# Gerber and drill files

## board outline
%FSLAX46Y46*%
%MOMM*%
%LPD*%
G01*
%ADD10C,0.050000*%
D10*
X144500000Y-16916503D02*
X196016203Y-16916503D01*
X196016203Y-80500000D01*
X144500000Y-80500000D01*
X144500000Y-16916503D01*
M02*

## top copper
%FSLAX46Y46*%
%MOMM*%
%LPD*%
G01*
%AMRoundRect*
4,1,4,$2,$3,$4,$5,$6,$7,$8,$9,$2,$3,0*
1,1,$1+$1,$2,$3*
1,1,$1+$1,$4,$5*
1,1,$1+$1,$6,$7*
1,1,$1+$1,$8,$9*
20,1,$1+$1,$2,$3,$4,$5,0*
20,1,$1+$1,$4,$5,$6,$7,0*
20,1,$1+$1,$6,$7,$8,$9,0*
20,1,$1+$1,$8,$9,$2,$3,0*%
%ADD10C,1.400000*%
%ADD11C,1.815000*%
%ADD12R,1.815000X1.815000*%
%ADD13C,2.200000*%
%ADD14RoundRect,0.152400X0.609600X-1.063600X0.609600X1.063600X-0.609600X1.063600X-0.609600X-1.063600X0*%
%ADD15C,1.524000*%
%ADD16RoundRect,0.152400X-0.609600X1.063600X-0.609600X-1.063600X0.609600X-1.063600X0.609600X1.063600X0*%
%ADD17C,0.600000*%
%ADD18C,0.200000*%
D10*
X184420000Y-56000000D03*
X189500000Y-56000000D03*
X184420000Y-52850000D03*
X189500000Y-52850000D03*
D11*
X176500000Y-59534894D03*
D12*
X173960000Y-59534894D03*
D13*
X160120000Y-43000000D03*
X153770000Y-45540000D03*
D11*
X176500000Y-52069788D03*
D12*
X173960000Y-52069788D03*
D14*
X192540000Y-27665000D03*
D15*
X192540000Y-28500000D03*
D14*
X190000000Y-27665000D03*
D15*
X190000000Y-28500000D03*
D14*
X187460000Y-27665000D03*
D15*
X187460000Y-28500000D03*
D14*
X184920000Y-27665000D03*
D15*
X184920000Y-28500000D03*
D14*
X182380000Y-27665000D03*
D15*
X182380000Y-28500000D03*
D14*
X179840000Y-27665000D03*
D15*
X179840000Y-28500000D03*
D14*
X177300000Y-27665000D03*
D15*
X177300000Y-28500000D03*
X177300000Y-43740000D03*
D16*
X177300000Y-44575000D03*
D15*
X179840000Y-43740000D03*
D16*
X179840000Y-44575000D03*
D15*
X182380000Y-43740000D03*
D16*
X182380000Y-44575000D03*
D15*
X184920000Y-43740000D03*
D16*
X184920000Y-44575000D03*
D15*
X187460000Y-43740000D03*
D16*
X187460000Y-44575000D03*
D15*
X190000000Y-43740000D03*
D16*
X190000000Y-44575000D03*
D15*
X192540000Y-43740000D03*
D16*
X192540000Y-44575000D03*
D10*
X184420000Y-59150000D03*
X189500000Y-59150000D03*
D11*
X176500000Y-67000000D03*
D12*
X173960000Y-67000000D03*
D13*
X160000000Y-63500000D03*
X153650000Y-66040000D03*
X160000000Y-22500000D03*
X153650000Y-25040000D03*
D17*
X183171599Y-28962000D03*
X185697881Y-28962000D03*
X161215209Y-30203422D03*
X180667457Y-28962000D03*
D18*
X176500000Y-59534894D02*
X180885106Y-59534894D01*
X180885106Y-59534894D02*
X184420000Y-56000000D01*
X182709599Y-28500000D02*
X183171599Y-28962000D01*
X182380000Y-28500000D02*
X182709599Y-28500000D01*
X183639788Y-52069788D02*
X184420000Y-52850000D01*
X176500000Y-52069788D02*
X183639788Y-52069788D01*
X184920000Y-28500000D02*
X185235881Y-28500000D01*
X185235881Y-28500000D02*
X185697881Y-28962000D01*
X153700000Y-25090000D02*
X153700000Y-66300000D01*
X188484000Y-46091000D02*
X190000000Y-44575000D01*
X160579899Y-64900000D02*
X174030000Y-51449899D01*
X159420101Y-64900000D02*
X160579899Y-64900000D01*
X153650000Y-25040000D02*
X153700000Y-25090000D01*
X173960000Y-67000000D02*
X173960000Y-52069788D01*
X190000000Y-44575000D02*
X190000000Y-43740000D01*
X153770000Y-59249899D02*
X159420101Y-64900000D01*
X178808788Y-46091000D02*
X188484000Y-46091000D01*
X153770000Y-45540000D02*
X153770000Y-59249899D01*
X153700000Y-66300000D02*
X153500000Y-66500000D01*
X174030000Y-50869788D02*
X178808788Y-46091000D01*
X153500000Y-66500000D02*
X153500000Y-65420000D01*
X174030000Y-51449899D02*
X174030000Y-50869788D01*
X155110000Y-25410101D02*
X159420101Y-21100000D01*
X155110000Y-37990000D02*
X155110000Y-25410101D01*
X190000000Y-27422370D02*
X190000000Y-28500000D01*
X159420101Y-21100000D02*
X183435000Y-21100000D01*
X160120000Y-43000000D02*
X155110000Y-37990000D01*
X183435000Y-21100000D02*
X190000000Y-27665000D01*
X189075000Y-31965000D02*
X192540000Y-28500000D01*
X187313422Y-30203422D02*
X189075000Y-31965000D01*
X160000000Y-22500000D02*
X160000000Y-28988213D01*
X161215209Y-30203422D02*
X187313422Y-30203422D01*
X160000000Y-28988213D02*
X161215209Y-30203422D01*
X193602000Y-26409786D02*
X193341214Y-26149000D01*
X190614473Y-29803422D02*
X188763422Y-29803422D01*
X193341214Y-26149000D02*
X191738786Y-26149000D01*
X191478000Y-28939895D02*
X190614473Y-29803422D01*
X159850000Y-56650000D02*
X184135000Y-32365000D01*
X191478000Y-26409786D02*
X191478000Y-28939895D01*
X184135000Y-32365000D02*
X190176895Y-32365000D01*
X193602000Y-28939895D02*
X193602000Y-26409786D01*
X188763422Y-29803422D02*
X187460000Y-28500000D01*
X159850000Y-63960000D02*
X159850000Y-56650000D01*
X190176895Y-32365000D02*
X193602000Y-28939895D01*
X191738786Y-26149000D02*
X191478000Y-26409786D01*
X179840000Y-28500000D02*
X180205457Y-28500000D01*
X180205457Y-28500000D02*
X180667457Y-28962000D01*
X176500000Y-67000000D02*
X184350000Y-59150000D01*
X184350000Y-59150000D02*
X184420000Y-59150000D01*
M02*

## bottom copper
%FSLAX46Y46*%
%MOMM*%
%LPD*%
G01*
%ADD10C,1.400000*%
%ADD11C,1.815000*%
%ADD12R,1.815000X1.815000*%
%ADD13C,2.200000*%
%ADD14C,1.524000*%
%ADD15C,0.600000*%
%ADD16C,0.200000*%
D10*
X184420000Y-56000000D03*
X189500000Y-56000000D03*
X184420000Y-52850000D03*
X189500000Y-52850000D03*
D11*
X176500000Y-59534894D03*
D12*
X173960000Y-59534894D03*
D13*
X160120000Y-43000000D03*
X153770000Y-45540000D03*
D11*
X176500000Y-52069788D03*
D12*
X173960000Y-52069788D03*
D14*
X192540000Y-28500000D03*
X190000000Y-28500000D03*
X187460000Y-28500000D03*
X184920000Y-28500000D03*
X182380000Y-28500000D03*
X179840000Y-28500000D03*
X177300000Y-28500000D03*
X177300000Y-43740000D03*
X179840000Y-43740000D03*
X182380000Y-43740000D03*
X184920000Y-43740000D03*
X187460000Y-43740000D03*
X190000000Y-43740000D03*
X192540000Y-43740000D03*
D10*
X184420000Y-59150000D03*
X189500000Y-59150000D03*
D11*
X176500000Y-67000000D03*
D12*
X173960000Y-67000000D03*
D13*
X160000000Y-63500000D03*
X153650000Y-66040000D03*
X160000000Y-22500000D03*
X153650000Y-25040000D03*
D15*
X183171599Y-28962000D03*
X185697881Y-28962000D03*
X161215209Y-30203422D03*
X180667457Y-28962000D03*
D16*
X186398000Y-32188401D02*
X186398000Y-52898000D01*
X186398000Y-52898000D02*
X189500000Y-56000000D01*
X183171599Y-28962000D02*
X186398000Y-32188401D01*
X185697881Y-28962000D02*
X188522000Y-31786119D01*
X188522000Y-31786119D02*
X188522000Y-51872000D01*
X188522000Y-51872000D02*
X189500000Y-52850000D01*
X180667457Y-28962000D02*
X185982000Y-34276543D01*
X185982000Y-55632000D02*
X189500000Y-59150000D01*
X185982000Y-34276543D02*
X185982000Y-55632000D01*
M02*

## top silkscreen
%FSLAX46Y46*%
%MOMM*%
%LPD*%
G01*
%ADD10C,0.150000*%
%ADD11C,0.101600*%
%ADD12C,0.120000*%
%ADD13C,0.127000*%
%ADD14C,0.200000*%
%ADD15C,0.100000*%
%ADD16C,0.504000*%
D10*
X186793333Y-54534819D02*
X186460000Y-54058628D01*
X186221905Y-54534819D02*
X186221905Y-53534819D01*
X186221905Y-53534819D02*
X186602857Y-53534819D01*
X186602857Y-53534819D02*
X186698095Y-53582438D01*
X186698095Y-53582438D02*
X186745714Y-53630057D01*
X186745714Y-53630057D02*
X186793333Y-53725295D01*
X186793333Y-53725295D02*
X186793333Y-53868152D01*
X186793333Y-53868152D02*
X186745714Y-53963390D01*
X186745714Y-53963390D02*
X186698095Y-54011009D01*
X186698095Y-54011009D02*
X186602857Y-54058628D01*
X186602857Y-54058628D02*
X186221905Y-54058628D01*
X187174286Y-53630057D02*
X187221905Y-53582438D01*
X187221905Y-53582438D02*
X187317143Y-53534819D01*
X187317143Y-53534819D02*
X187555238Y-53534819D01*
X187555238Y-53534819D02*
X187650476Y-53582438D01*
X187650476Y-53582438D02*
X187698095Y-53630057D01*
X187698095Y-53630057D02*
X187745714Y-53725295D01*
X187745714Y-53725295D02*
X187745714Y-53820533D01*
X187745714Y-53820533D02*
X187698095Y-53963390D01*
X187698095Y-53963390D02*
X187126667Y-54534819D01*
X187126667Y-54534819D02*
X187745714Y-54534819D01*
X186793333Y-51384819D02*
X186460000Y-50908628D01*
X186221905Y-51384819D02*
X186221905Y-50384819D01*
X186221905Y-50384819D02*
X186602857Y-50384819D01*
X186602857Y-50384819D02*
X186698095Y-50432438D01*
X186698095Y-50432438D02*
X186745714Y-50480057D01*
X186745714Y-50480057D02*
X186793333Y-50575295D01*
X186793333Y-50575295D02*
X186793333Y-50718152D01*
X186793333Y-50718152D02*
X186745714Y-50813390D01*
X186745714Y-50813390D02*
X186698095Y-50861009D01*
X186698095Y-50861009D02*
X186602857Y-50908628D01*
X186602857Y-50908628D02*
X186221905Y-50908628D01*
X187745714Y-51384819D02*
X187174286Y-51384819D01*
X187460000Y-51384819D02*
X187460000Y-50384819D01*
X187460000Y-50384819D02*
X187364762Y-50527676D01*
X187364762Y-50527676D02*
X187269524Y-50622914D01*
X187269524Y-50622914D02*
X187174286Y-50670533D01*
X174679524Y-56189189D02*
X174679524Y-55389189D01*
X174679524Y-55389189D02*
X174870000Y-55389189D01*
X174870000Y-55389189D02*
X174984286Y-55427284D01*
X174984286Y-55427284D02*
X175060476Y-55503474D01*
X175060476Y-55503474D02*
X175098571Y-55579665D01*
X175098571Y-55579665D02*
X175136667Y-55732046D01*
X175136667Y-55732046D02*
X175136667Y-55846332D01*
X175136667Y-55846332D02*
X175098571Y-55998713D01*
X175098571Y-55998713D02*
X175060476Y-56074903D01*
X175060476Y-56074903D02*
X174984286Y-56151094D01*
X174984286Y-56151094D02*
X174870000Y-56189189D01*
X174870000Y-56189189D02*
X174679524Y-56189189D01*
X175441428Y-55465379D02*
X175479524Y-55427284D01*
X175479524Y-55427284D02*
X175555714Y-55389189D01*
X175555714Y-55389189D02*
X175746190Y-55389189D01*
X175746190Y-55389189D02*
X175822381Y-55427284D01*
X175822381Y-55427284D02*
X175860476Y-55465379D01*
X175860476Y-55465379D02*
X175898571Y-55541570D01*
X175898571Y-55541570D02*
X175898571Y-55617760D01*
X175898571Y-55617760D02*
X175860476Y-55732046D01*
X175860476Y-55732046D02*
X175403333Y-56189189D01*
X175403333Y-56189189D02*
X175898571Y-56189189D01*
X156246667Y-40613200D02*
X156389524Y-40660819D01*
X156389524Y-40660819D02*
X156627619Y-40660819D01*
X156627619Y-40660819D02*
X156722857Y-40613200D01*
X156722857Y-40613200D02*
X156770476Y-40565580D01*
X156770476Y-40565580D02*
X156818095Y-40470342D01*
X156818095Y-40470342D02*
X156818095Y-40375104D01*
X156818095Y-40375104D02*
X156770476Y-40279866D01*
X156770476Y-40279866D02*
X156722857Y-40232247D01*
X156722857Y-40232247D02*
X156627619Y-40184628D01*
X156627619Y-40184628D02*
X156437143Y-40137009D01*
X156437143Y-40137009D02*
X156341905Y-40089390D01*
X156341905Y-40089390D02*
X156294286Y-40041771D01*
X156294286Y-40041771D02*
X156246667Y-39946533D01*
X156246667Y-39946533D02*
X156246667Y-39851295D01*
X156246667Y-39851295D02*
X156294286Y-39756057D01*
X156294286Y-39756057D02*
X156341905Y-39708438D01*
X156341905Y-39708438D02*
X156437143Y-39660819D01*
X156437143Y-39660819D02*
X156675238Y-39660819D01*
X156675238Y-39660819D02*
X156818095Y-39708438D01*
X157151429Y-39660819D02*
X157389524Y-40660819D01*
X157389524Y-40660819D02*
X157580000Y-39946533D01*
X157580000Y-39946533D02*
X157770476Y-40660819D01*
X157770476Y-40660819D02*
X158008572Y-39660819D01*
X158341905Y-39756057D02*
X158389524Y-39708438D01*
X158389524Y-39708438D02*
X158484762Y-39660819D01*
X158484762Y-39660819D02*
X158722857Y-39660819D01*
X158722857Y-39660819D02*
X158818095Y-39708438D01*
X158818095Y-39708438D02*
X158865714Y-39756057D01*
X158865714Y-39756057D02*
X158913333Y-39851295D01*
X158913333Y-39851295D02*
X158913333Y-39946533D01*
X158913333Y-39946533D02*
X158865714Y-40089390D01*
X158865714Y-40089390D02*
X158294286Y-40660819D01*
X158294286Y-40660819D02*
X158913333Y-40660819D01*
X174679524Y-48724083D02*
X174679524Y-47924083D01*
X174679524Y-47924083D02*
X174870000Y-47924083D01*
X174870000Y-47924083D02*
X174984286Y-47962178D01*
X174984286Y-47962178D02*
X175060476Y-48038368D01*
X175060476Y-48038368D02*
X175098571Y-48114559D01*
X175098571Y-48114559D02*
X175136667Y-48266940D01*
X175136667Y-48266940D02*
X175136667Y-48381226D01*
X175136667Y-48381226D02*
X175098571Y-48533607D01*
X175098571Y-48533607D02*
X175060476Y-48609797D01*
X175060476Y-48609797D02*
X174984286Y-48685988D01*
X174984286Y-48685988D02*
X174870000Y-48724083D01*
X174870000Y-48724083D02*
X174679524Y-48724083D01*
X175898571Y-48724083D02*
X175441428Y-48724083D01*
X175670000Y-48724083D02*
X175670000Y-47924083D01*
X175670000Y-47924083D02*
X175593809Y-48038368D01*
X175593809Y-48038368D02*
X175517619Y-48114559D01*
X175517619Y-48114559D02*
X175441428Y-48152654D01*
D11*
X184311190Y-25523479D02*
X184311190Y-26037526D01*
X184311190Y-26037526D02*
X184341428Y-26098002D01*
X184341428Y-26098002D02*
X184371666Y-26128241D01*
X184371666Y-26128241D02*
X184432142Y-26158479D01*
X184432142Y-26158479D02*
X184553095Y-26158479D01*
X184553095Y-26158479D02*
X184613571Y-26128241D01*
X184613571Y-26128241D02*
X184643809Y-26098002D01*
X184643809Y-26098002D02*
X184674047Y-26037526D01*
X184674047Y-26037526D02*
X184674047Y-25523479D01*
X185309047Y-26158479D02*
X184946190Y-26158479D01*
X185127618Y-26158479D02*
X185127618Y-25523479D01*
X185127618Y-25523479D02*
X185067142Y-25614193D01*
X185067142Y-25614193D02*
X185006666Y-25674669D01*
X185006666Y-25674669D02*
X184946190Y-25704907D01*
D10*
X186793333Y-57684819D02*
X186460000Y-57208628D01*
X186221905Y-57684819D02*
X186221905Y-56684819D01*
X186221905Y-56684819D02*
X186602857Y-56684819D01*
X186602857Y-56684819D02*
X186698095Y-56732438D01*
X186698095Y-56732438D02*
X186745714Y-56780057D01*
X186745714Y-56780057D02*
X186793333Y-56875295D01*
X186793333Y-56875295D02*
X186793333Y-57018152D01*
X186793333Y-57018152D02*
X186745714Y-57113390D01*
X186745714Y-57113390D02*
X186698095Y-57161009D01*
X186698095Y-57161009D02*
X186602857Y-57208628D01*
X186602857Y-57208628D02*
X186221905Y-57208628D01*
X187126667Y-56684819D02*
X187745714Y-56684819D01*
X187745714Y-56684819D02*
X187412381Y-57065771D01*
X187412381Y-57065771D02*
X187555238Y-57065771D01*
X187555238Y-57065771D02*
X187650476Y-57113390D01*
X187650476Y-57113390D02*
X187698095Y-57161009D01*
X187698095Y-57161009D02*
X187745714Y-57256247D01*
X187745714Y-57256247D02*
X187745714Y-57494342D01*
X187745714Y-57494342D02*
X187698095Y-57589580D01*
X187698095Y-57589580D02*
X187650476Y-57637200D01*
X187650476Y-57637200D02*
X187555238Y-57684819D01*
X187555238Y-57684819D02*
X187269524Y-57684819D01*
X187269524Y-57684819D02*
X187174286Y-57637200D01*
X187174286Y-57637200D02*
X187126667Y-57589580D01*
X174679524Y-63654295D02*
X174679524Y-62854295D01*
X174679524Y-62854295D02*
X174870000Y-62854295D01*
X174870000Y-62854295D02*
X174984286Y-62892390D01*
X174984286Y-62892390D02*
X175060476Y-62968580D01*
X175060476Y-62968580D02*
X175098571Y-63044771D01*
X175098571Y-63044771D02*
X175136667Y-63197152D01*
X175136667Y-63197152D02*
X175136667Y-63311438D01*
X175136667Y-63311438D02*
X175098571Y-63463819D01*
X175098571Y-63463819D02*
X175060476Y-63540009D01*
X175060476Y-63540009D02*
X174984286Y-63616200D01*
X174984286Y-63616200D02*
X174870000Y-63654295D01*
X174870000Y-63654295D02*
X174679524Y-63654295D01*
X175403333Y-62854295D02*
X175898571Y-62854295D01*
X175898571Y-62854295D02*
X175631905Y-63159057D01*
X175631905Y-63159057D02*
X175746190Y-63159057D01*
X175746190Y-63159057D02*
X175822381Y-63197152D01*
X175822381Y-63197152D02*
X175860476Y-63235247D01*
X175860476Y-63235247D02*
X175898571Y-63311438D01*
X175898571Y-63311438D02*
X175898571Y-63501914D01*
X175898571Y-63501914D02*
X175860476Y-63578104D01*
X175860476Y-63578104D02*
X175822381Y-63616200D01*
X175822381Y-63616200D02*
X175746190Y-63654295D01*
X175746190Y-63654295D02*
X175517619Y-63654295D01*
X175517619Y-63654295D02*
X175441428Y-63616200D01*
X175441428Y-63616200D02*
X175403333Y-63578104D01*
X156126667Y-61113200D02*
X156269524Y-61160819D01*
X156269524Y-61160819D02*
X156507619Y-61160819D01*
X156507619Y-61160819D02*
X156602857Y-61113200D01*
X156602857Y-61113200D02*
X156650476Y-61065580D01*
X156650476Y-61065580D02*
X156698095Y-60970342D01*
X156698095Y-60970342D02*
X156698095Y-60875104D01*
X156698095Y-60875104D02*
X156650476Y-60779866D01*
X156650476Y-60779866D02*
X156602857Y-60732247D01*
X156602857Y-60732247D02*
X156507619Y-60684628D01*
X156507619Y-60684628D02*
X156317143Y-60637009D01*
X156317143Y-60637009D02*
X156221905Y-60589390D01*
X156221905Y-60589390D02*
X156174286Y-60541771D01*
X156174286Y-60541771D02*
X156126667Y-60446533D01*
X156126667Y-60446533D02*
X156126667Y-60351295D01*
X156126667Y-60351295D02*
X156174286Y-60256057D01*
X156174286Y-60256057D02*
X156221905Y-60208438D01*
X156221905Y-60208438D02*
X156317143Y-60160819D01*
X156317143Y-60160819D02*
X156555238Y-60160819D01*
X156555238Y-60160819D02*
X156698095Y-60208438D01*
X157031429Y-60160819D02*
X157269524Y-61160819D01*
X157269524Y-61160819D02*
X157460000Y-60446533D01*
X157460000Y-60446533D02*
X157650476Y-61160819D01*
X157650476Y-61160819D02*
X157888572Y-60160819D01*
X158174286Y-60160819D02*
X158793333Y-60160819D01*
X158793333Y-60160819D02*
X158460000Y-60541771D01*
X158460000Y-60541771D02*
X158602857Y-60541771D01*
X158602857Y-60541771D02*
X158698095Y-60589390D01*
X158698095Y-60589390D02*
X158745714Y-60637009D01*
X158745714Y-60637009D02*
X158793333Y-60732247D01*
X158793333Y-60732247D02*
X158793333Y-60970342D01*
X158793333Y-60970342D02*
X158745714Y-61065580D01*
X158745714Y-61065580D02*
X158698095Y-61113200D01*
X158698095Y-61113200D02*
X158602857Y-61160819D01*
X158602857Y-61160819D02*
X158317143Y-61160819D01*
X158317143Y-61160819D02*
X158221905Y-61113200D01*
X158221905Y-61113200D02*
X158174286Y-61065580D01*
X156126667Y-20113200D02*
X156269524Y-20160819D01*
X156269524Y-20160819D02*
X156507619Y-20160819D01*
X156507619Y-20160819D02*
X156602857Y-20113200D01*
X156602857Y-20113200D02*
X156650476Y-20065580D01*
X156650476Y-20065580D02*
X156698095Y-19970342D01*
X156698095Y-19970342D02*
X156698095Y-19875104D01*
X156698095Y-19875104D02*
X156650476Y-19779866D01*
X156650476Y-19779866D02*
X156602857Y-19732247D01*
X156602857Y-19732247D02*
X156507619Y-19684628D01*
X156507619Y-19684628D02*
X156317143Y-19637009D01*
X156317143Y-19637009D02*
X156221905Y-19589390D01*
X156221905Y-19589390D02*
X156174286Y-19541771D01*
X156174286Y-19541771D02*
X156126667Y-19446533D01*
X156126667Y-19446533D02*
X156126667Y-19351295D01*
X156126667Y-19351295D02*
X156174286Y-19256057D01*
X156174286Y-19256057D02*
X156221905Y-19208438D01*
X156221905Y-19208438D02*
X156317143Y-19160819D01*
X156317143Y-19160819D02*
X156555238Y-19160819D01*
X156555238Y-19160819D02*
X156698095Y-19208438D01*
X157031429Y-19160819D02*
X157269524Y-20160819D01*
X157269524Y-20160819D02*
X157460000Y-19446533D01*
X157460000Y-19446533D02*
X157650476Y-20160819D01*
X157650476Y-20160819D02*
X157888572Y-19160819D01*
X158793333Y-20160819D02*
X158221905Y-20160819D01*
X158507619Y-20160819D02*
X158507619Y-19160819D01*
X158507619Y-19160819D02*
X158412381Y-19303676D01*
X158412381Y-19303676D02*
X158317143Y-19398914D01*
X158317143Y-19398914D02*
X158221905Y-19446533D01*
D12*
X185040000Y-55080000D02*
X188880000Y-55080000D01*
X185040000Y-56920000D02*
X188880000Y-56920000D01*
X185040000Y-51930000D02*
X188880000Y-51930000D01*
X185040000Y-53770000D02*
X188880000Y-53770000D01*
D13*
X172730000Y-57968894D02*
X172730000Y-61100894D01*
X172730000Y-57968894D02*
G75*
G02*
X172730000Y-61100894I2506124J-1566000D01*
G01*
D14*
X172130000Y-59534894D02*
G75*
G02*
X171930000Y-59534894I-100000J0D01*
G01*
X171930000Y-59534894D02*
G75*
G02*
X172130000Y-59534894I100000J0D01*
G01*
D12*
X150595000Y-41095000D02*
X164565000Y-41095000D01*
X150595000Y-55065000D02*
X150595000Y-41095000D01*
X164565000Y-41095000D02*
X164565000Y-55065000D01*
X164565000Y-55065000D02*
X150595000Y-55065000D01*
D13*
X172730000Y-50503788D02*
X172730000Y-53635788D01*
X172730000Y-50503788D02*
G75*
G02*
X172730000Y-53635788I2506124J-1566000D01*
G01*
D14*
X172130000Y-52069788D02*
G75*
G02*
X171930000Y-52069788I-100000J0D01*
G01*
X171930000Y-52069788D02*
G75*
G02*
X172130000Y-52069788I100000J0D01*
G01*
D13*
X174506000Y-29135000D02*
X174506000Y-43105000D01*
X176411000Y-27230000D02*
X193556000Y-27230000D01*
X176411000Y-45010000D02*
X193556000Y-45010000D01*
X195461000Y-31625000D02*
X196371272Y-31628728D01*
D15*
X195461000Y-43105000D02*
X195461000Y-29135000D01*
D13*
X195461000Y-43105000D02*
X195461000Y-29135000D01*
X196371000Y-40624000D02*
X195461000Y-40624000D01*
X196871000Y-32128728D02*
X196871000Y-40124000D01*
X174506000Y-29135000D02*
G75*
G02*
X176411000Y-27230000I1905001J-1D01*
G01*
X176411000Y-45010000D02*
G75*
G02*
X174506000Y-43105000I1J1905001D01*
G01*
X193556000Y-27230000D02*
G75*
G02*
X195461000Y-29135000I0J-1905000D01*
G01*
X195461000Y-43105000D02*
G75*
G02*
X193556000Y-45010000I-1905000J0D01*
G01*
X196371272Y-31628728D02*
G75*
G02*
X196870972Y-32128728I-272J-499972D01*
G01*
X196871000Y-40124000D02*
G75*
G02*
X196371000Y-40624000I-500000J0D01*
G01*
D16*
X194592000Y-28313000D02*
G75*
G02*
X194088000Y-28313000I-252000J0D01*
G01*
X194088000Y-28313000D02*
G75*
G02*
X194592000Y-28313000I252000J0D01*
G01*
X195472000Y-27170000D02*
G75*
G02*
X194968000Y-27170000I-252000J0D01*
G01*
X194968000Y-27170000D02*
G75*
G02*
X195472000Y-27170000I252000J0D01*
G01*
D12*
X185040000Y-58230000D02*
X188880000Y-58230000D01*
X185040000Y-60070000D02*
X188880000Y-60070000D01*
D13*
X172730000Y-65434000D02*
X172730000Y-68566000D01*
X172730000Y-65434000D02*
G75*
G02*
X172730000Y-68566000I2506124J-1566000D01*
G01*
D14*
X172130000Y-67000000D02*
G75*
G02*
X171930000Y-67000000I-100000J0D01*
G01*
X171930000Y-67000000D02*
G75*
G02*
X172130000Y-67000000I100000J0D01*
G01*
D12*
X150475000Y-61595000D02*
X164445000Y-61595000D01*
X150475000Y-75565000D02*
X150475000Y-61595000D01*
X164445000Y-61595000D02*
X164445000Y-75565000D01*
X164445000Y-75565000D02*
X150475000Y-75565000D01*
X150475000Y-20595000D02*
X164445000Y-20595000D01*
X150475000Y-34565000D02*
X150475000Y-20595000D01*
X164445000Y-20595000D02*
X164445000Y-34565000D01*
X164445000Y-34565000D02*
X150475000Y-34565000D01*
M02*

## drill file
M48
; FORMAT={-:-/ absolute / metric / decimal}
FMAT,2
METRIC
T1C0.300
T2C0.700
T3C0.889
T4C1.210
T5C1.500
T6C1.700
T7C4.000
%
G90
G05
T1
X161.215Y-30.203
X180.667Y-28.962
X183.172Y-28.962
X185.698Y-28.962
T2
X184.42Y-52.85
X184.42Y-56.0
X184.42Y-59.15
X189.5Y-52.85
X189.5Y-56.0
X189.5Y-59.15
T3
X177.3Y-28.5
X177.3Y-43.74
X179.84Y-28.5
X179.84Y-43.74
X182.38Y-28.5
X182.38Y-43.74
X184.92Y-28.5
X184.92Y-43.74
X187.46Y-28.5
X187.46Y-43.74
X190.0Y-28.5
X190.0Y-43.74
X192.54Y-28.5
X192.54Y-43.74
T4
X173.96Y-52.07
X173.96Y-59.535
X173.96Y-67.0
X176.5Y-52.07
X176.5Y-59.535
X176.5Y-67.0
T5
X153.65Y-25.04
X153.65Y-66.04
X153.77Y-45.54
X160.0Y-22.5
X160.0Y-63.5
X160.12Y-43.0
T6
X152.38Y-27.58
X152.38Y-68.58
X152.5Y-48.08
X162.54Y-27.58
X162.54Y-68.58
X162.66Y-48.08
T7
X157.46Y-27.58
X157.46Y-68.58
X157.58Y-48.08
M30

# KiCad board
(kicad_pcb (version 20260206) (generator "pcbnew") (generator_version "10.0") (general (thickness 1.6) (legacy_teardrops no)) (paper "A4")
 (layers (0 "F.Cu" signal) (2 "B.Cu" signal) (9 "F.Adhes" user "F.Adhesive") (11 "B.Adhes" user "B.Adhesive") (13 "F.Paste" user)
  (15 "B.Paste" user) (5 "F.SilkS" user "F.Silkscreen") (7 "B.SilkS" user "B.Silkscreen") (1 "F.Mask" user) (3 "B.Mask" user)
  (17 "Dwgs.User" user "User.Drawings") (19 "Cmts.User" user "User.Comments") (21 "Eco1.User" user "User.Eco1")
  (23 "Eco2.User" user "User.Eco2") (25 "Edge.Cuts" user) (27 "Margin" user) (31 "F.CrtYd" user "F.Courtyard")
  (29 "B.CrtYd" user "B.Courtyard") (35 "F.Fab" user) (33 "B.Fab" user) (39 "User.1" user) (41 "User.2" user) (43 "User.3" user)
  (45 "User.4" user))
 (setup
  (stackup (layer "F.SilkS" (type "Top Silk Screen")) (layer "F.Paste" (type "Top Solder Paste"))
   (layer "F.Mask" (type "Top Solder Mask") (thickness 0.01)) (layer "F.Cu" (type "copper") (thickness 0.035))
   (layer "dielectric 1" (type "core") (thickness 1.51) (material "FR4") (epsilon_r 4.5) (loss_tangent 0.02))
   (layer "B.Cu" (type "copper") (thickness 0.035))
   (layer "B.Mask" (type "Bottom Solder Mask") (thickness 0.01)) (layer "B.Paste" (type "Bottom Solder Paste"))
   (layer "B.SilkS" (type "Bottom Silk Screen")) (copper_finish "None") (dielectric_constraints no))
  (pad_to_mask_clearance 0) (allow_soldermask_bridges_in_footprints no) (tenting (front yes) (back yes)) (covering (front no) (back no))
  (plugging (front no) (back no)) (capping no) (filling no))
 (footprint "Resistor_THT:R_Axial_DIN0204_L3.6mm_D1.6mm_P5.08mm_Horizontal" (layer "F.Cu") (at 184.42 56)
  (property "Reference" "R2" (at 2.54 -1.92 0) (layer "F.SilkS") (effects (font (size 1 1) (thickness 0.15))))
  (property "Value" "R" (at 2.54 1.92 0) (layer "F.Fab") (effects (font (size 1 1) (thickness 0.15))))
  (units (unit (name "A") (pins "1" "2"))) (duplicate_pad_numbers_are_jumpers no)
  (fp_line (start 0.62 -0.92) (end 4.46 -0.92) (stroke (width 0.12) (type solid)) (layer "F.SilkS"))
  (fp_line (start 0.62 0.92) (end 4.46 0.92) (stroke (width 0.12) (type solid)) (layer "F.SilkS"))
  (pad "1" thru_hole circle (at 0 0) (size 1.4 1.4) (drill 0.7) (layers "*.Cu" "*.Mask") (remove_unused_layers no) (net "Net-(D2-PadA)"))
  (pad "2" thru_hole circle (at 5.08 0) (size 1.4 1.4) (drill 0.7) (layers "*.Cu" "*.Mask") (remove_unused_layers no) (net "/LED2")))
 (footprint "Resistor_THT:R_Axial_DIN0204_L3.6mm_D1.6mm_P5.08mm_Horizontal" (layer "F.Cu") (at 184.42 52.85)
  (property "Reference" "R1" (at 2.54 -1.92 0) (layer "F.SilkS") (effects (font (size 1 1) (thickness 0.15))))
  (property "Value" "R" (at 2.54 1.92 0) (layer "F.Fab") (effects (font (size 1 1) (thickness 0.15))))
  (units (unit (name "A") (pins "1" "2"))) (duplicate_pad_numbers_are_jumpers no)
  (fp_line (start 0.62 -0.92) (end 4.46 -0.92) (stroke (width 0.12) (type solid)) (layer "F.SilkS"))
  (fp_line (start 0.62 0.92) (end 4.46 0.92) (stroke (width 0.12) (type solid)) (layer "F.SilkS"))
  (pad "1" thru_hole circle (at 0 0) (size 1.4 1.4) (drill 0.7) (layers "*.Cu" "*.Mask") (remove_unused_layers no) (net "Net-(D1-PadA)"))
  (pad "2" thru_hole circle (at 5.08 0) (size 1.4 1.4) (drill 0.7) (layers "*.Cu" "*.Mask") (remove_unused_layers no) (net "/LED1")))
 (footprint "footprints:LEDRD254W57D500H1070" (layer "F.Cu") (at 175.23 59.534894)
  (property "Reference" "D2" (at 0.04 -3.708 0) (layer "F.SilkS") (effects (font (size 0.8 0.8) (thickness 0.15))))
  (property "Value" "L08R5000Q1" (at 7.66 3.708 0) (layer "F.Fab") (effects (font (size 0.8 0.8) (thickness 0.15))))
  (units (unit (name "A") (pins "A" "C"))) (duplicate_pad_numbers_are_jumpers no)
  (fp_line (start -2.5 -1.566) (end -2.5 1.566) (stroke (width 0.127) (type solid)) (layer "F.SilkS"))
  (fp_arc (start -2.5 -1.566) (mid 2.961291 0) (end -2.5 1.566) (stroke (width 0.127) (type solid)) (layer "F.SilkS"))
  (fp_circle (center -3.2 0) (end -3.1 0) (stroke (width 0.2) (type solid)) (fill no) (layer "F.SilkS"))
  (pad "A" thru_hole circle (at 1.27 0) (size 1.815 1.815) (drill 1.21) (layers "*.Cu" "*.Mask") (remove_unused_layers no)
   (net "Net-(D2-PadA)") (solder_mask_margin 0.102))
  (pad "C" thru_hole rect (at -1.27 0) (size 1.815 1.815) (drill 1.21) (layers "*.Cu" "*.Mask") (remove_unused_layers no) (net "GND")
   (solder_mask_margin 0.102)))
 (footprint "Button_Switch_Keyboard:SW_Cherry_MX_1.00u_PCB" (layer "F.Cu") (at 160.12 43)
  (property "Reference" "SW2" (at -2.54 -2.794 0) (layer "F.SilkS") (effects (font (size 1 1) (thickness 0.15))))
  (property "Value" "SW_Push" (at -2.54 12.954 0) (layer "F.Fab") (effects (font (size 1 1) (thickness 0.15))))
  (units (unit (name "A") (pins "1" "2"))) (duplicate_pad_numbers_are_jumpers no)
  (fp_line (start -9.525 -1.905) (end 4.445 -1.905) (stroke (width 0.12) (type solid)) (layer "F.SilkS"))
  (fp_line (start -9.525 12.065) (end -9.525 -1.905) (stroke (width 0.12) (type solid)) (layer "F.SilkS"))
  (fp_line (start 4.445 -1.905) (end 4.445 12.065) (stroke (width 0.12) (type solid)) (layer "F.SilkS"))
  (fp_line (start 4.445 12.065) (end -9.525 12.065) (stroke (width 0.12) (type solid)) (layer "F.SilkS"))
  (pad "" np_thru_hole circle (at -7.62 5.08) (size 1.7 1.7) (drill 1.7) (layers "*.Cu" "*.Mask"))
  (pad "" np_thru_hole circle (at -2.54 5.08) (size 4 4) (drill 4) (layers "*.Cu" "*.Mask"))
  (pad "" np_thru_hole circle (at 2.54 5.08) (size 1.7 1.7) (drill 1.7) (layers "*.Cu" "*.Mask"))
  (pad "1" thru_hole circle (at 0 0) (size 2.2 2.2) (drill 1.5) (layers "*.Cu" "*.Mask") (remove_unused_layers no) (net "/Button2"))
  (pad "2" thru_hole circle (at -6.35 2.54) (size 2.2 2.2) (drill 1.5) (layers "*.Cu" "*.Mask") (remove_unused_layers no) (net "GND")))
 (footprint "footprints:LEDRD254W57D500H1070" (layer "F.Cu") (at 175.23 52.069788)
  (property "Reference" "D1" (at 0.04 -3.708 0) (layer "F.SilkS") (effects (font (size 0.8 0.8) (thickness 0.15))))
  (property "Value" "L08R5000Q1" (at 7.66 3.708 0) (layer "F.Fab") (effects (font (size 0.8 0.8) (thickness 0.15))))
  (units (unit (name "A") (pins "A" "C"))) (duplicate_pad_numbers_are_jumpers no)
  (fp_line (start -2.5 -1.566) (end -2.5 1.566) (stroke (width 0.127) (type solid)) (layer "F.SilkS"))
  (fp_arc (start -2.5 -1.566) (mid 2.961291 0) (end -2.5 1.566) (stroke (width 0.127) (type solid)) (layer "F.SilkS"))
  (fp_circle (center -3.2 0) (end -3.1 0) (stroke (width 0.2) (type solid)) (fill no) (layer "F.SilkS"))
  (pad "A" thru_hole circle (at 1.27 0) (size 1.815 1.815) (drill 1.21) (layers "*.Cu" "*.Mask") (remove_unused_layers no)
   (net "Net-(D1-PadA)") (solder_mask_margin 0.102))
  (pad "C" thru_hole rect (at -1.27 0) (size 1.815 1.815) (drill 1.21) (layers "*.Cu" "*.Mask") (remove_unused_layers no) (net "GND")
   (solder_mask_margin 0.102)))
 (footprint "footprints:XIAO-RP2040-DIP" (layer "F.Cu") (at 184.92 36.12)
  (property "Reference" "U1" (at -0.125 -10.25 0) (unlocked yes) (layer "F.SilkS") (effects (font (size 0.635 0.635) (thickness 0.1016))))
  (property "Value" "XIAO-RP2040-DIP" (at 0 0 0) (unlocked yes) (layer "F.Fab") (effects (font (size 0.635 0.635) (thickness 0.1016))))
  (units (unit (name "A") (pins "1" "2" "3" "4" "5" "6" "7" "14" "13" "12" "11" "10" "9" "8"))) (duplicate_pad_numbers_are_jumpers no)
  (fp_line (start -10.414 -6.985) (end -10.414 6.985) (stroke (width 0.127) (type solid)) (layer "F.SilkS"))
  (fp_line (start -8.509 -8.89) (end 8.636 -8.89) (stroke (width 0.127) (type solid)) (layer "F.SilkS"))
  (fp_line (start -8.509 8.89) (end 8.636 8.89) (stroke (width 0.127) (type solid)) (layer "F.SilkS"))
  (fp_line (start 10.541 -4.495) (end 11.451272 -4.491272) (stroke (width 0.127) (type solid)) (layer "F.SilkS"))
  (fp_line (start 10.541 6.985) (end 10.541 -6.985) (stroke (width 0.1) (type solid)) (layer "F.SilkS"))
  (fp_line (start 10.541 6.985) (end 10.541 -6.985) (stroke (width 0.127) (type solid)) (layer "F.SilkS"))
  (fp_line (start 11.451 4.504) (end 10.541 4.504) (stroke (width 0.127) (type solid)) (layer "F.SilkS"))
  (fp_line (start 11.951 -3.991272) (end 11.951 4.004) (stroke (width 0.127) (type solid)) (layer "F.SilkS"))
  (fp_arc (start -10.414 -6.985) (mid -9.856038 -8.332038) (end -8.509 -8.89) (stroke (width 0.127) (type solid)) (layer "F.SilkS"))
  (fp_arc (start -8.509 8.89) (mid -9.856038 8.332038) (end -10.414 6.985) (stroke (width 0.127) (type solid)) (layer "F.SilkS"))
  (fp_arc (start 8.636 -8.89) (mid 9.983038 -8.332038) (end 10.541 -6.985) (stroke (width 0.127) (type solid)) (layer "F.SilkS"))
  (fp_arc (start 10.541 6.985) (mid 9.983038 8.332038) (end 8.636 8.89) (stroke (width 0.127) (type solid)) (layer "F.SilkS"))
  (fp_arc (start 11.451272 -4.491272) (mid 11.804644 -4.344724) (end 11.951 -3.991272) (stroke (width 0.127) (type default))
   (layer "F.SilkS"))
  (fp_arc (start 11.951 4.004) (mid 11.804553 4.357553) (end 11.451 4.504) (stroke (width 0.127) (type default)) (layer "F.SilkS"))
  (fp_circle (center 9.42 -7.807) (end 9.674 -7.807) (stroke (width 0.5) (type solid)) (fill yes) (layer "F.SilkS"))
  (fp_circle (center 10.3 -8.95) (end 10.554 -8.95) (stroke (width 0.5) (type solid)) (fill yes) (layer "F.SilkS"))
  (pad "1" smd roundrect (at 7.62 -8.455 90) (size 2.432 1.524) (layers "F.Cu" "F.Mask") (roundrect_rratio 0.1) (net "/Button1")
   (thermal_bridge_angle 45))
  (pad "1" thru_hole circle (at 7.62 -7.62 90) (size 1.524 1.524) (drill 0.889) (layers "*.Cu" "*.Mask") (remove_unused_layers no)
   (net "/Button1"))
  (pad "2" smd roundrect (at 5.08 -8.455 90) (size 2.432 1.524) (layers "F.Cu" "F.Mask") (roundrect_rratio 0.1) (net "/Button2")
   (thermal_bridge_angle 45))
  (pad "2" thru_hole circle (at 5.08 -7.62 90) (size 1.524 1.524) (drill 0.889) (layers "*.Cu" "*.Mask") (remove_unused_layers no)
   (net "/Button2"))
  (pad "3" smd roundrect (at 2.54 -8.455 90) (size 2.432 1.524) (layers "F.Cu" "F.Mask") (roundrect_rratio 0.1) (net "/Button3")
   (thermal_bridge_angle 45))
  (pad "3" thru_hole circle (at 2.54 -7.62 90) (size 1.524 1.524) (drill 0.889) (layers "*.Cu" "*.Mask") (remove_unused_layers no)
   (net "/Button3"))
  (pad "4" smd roundrect (at 0 -8.455 90) (size 2.432 1.524) (layers "F.Cu" "F.Mask") (roundrect_rratio 0.1) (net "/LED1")
   (thermal_bridge_angle 45))
  (pad "4" thru_hole circle (at 0 -7.62 90) (size 1.524 1.524) (drill 0.889) (layers "*.Cu" "*.Mask") (remove_unused_layers no)
   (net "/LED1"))
  (pad "5" smd roundrect (at -2.54 -8.455 90) (size 2.432 1.524) (layers "F.Cu" "F.Mask") (roundrect_rratio 0.1) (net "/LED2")
   (thermal_bridge_angle 45))
  (pad "5" thru_hole circle (at -2.54 -7.62 90) (size 1.524 1.524) (drill 0.889) (layers "*.Cu" "*.Mask") (remove_unused_layers no)
   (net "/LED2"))
  (pad "6" smd roundrect (at -5.08 -8.455 90) (size 2.432 1.524) (layers "F.Cu" "F.Mask") (roundrect_rratio 0.1) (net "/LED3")
   (thermal_bridge_angle 45))
  (pad "6" thru_hole circle (at -5.08 -7.62 90) (size 1.524 1.524) (drill 0.889) (layers "*.Cu" "*.Mask") (remove_unused_layers no)
   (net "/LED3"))
  (pad "7" smd roundrect (at -7.62 -8.455 90) (size 2.432 1.524) (layers "F.Cu" "F.Mask") (roundrect_rratio 0.1)
   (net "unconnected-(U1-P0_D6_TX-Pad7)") (thermal_bridge_angle 45))
  (pad "7" thru_hole circle (at -7.62 -7.62 90) (size 1.524 1.524) (drill 0.889) (layers "*.Cu" "*.Mask") (remove_unused_layers no)
   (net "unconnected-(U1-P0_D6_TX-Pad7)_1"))
  (pad "8" thru_hole circle (at -7.62 7.62 270) (size 1.524 1.524) (drill 0.889) (layers "*.Cu" "*.Mask") (remove_unused_layers no)
   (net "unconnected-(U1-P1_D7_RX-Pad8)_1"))
  (pad "8" smd roundrect (at -7.62 8.455 270) (size 2.432 1.524) (layers "F.Cu" "F.Mask") (roundrect_rratio 0.1)
   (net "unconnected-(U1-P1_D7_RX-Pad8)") (thermal_bridge_angle 45))
  (pad "9" thru_hole circle (at -5.08 7.62 270) (size 1.524 1.524) (drill 0.889) (layers "*.Cu" "*.Mask") (remove_unused_layers no)
   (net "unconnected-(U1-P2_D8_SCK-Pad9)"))
  (pad "9" smd roundrect (at -5.08 8.455 270) (size 2.432 1.524) (layers "F.Cu" "F.Mask") (roundrect_rratio 0.1)
   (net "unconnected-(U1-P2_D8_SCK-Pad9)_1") (thermal_bridge_angle 45))
  (pad "10" thru_hole circle (at -2.54 7.62 270) (size 1.524 1.524) (drill 0.889) (layers "*.Cu" "*.Mask") (remove_unused_layers no)
   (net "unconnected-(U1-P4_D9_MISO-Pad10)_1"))
  (pad "10" smd roundrect (at -2.54 8.455 270) (size 2.432 1.524) (layers "F.Cu" "F.Mask") (roundrect_rratio 0.1)
   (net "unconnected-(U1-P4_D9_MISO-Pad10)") (thermal_bridge_angle 45))
  (pad "11" thru_hole circle (at 0 7.62 270) (size 1.524 1.524) (drill 0.889) (layers "*.Cu" "*.Mask") (remove_unused_layers no)
   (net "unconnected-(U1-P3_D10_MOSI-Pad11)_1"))
  (pad "11" smd roundrect (at 0 8.455 270) (size 2.432 1.524) (layers "F.Cu" "F.Mask") (roundrect_rratio 0.1)
   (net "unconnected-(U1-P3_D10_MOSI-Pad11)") (thermal_bridge_angle 45))
  (pad "12" thru_hole circle (at 2.54 7.62 270) (size 1.524 1.524) (drill 0.889) (layers "*.Cu" "*.Mask") (remove_unused_layers no)
   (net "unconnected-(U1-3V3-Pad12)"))
  (pad "12" smd roundrect (at 2.54 8.455 270) (size 2.432 1.524) (layers "F.Cu" "F.Mask") (roundrect_rratio 0.1)
   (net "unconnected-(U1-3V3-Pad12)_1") (thermal_bridge_angle 45))
  (pad "13" thru_hole circle (at 5.08 7.62 270) (size 1.524 1.524) (drill 0.889) (layers "*.Cu" "*.Mask") (remove_unused_layers no)
   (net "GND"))
  (pad "13" smd roundrect (at 5.08 8.455 270) (size 2.432 1.524) (layers "F.Cu" "F.Mask") (roundrect_rratio 0.1) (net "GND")
   (thermal_bridge_angle 45))
  (pad "14" thru_hole circle (at 7.62 7.62 270) (size 1.524 1.524) (drill 0.889) (layers "*.Cu" "*.Mask") (remove_unused_layers no)
   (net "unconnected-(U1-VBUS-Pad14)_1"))
  (pad "14" smd roundrect (at 7.62 8.455 270) (size 2.432 1.524) (layers "F.Cu" "F.Mask") (roundrect_rratio 0.1)
   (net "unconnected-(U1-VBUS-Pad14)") (thermal_bridge_angle 45)))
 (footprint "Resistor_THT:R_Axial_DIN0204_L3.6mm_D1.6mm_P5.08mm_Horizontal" (layer "F.Cu") (at 184.42 59.15)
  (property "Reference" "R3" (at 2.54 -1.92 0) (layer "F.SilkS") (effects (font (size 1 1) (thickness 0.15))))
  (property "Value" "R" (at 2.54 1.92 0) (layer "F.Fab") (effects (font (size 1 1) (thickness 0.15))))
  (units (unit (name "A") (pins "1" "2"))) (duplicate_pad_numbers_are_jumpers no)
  (fp_line (start 0.62 -0.92) (end 4.46 -0.92) (stroke (width 0.12) (type solid)) (layer "F.SilkS"))
  (fp_line (start 0.62 0.92) (end 4.46 0.92) (stroke (width 0.12) (type solid)) (layer "F.SilkS"))
  (pad "1" thru_hole circle (at 0 0) (size 1.4 1.4) (drill 0.7) (layers "*.Cu" "*.Mask") (remove_unused_layers no) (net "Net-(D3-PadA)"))
  (pad "2" thru_hole circle (at 5.08 0) (size 1.4 1.4) (drill 0.7) (layers "*.Cu" "*.Mask") (remove_unused_layers no) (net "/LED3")))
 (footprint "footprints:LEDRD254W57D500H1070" (layer "F.Cu") (at 175.23 67)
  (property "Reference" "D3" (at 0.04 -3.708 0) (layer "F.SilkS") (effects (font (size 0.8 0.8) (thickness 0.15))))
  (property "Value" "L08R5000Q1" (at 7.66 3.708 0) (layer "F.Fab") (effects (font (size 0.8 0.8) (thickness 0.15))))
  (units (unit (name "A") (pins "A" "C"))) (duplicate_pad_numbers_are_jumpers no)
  (fp_line (start -2.5 -1.566) (end -2.5 1.566) (stroke (width 0.127) (type solid)) (layer "F.SilkS"))
  (fp_arc (start -2.5 -1.566) (mid 2.961291 0) (end -2.5 1.566) (stroke (width 0.127) (type solid)) (layer "F.SilkS"))
  (fp_circle (center -3.2 0) (end -3.1 0) (stroke (width 0.2) (type solid)) (fill no) (layer "F.SilkS"))
  (pad "A" thru_hole circle (at 1.27 0) (size 1.815 1.815) (drill 1.21) (layers "*.Cu" "*.Mask") (remove_unused_layers no)
   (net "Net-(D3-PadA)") (solder_mask_margin 0.102))
  (pad "C" thru_hole rect (at -1.27 0) (size 1.815 1.815) (drill 1.21) (layers "*.Cu" "*.Mask") (remove_unused_layers no) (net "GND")
   (solder_mask_margin 0.102)))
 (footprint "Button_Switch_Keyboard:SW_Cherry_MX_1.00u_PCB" (layer "F.Cu") (at 160 63.5)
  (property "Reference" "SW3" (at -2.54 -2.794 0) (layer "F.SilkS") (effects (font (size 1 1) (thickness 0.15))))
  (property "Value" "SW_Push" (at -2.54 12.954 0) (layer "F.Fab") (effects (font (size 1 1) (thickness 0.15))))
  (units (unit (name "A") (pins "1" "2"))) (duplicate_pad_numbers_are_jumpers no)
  (fp_line (start -9.525 -1.905) (end 4.445 -1.905) (stroke (width 0.12) (type solid)) (layer "F.SilkS"))
  (fp_line (start -9.525 12.065) (end -9.525 -1.905) (stroke (width 0.12) (type solid)) (layer "F.SilkS"))
  (fp_line (start 4.445 -1.905) (end 4.445 12.065) (stroke (width 0.12) (type solid)) (layer "F.SilkS"))
  (fp_line (start 4.445 12.065) (end -9.525 12.065) (stroke (width 0.12) (type solid)) (layer "F.SilkS"))
  (pad "" np_thru_hole circle (at -7.62 5.08) (size 1.7 1.7) (drill 1.7) (layers "*.Cu" "*.Mask"))
  (pad "" np_thru_hole circle (at -2.54 5.08) (size 4 4) (drill 4) (layers "*.Cu" "*.Mask"))
  (pad "" np_thru_hole circle (at 2.54 5.08) (size 1.7 1.7) (drill 1.7) (layers "*.Cu" "*.Mask"))
  (pad "1" thru_hole circle (at 0 0) (size 2.2 2.2) (drill 1.5) (layers "*.Cu" "*.Mask") (remove_unused_layers no) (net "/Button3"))
  (pad "2" thru_hole circle (at -6.35 2.54) (size 2.2 2.2) (drill 1.5) (layers "*.Cu" "*.Mask") (remove_unused_layers no) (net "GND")))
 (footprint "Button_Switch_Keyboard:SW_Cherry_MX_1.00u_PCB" (layer "F.Cu") (at 160 22.5)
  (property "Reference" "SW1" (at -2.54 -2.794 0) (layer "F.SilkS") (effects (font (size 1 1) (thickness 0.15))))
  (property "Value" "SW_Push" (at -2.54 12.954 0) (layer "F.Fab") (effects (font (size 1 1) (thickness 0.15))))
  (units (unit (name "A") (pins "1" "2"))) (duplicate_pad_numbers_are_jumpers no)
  (fp_line (start -9.525 -1.905) (end 4.445 -1.905) (stroke (width 0.12) (type solid)) (layer "F.SilkS"))
  (fp_line (start -9.525 12.065) (end -9.525 -1.905) (stroke (width 0.12) (type solid)) (layer "F.SilkS"))
  (fp_line (start 4.445 -1.905) (end 4.445 12.065) (stroke (width 0.12) (type solid)) (layer "F.SilkS"))
  (fp_line (start 4.445 12.065) (end -9.525 12.065) (stroke (width 0.12) (type solid)) (layer "F.SilkS"))
  (pad "" np_thru_hole circle (at -7.62 5.08) (size 1.7 1.7) (drill 1.7) (layers "*.Cu" "*.Mask"))
  (pad "" np_thru_hole circle (at -2.54 5.08) (size 4 4) (drill 4) (layers "*.Cu" "*.Mask"))
  (pad "" np_thru_hole circle (at 2.54 5.08) (size 1.7 1.7) (drill 1.7) (layers "*.Cu" "*.Mask"))
  (pad "1" thru_hole circle (at 0 0) (size 2.2 2.2) (drill 1.5) (layers "*.Cu" "*.Mask") (remove_unused_layers no) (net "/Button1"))
  (pad "2" thru_hole circle (at -6.35 2.54) (size 2.2 2.2) (drill 1.5) (layers "*.Cu" "*.Mask") (remove_unused_layers no) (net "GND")))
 (gr_rect (start 144.5 16.916503) (end 196.016203 80.5) (stroke (width 0.05) (type default)) (fill no) (layer "Edge.Cuts"))
 (segment (start 176.5 59.534894) (end 180.885106 59.534894) (width 0.2) (layer "F.Cu") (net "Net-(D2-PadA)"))
 (segment (start 180.885106 59.534894) (end 184.42 56) (width 0.2) (layer "F.Cu") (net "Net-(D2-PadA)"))
 (segment (start 182.709599 28.5) (end 183.171599 28.962) (width 0.2) (layer "F.Cu") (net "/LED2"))
 (segment (start 182.38 28.5) (end 182.709599 28.5) (width 0.2) (layer "F.Cu") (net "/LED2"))
 (via (at 183.171599 28.962) (size 0.6) (drill 0.3) (layers "F.Cu" "B.Cu") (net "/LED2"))
 (segment (start 186.398 32.188401) (end 186.398 52.898) (width 0.2) (layer "B.Cu") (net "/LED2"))
 (segment (start 186.398 52.898) (end 189.5 56) (width 0.2) (layer "B.Cu") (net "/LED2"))
 (segment (start 183.171599 28.962) (end 186.398 32.188401) (width 0.2) (layer "B.Cu") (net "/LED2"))
 (segment (start 183.639788 52.069788) (end 184.42 52.85) (width 0.2) (layer "F.Cu") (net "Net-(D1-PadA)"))
 (segment (start 176.5 52.069788) (end 183.639788 52.069788) (width 0.2) (layer "F.Cu") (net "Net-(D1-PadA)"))
 (segment (start 184.92 28.5) (end 185.235881 28.5) (width 0.2) (layer "F.Cu") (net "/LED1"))
 (segment (start 185.235881 28.5) (end 185.697881 28.962) (width 0.2) (layer "F.Cu") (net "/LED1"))
 (via (at 185.697881 28.962) (size 0.6) (drill 0.3) (layers "F.Cu" "B.Cu") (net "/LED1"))
 (segment (start 185.697881 28.962) (end 188.522 31.786119) (width 0.2) (layer "B.Cu") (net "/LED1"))
 (segment (start 188.522 31.786119) (end 188.522 51.872) (width 0.2) (layer "B.Cu") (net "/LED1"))
 (segment (start 188.522 51.872) (end 189.5 52.85) (width 0.2) (layer "B.Cu") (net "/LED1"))
 (segment (start 153.7 25.09) (end 153.7 66.3) (width 0.2) (layer "F.Cu") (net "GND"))
 (segment (start 188.484 46.091) (end 190 44.575) (width 0.2) (layer "F.Cu") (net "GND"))
 (segment (start 160.579899 64.9) (end 174.03 51.449899) (width 0.2) (layer "F.Cu") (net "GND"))
 (segment (start 159.420101 64.9) (end 160.579899 64.9) (width 0.2) (layer "F.Cu") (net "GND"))
 (segment (start 153.65 25.04) (end 153.7 25.09) (width 0.2) (layer "F.Cu") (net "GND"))
 (segment (start 173.96 67) (end 173.96 52.069788) (width 0.2) (layer "F.Cu") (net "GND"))
 (segment (start 190 44.575) (end 190 43.74) (width 0.2) (layer "F.Cu") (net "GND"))
 (segment (start 153.77 59.249899) (end 159.420101 64.9) (width 0.2) (layer "F.Cu") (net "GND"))
 (segment (start 178.808788 46.091) (end 188.484 46.091) (width 0.2) (layer "F.Cu") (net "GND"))
 (segment (start 153.77 45.54) (end 153.77 59.249899) (width 0.2) (layer "F.Cu") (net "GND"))
 (segment (start 153.7 66.3) (end 153.5 66.5) (width 0.2) (layer "F.Cu") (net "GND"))
 (segment (start 174.03 50.869788) (end 178.808788 46.091) (width 0.2) (layer "F.Cu") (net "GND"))
 (segment (start 153.5 66.5) (end 153.5 65.42) (width 0.2) (layer "F.Cu") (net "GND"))
 (segment (start 174.03 51.449899) (end 174.03 50.869788) (width 0.2) (layer "F.Cu") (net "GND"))
 (segment (start 155.11 25.410101) (end 159.420101 21.1) (width 0.2) (layer "F.Cu") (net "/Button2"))
 (segment (start 155.11 37.99) (end 155.11 25.410101) (width 0.2) (layer "F.Cu") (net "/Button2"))
 (segment (start 190 27.42237) (end 190 28.5) (width 0.2) (layer "F.Cu") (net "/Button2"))
 (segment (start 159.420101 21.1) (end 183.435 21.1) (width 0.2) (layer "F.Cu") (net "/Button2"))
 (segment (start 160.12 43) (end 155.11 37.99) (width 0.2) (layer "F.Cu") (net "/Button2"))
 (segment (start 183.435 21.1) (end 190 27.665) (width 0.2) (layer "F.Cu") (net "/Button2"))
 (segment (start 189.075 31.965) (end 192.54 28.5) (width 0.2) (layer "F.Cu") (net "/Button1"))
 (segment (start 187.313422 30.203422) (end 189.075 31.965) (width 0.2) (layer "F.Cu") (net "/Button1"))
 (segment (start 160 22.5) (end 160 28.988213) (width 0.2) (layer "F.Cu") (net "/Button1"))
 (segment (start 161.215209 30.203422) (end 187.313422 30.203422) (width 0.2) (layer "F.Cu") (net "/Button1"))
 (segment (start 160 28.988213) (end 161.215209 30.203422) (width 0.2) (layer "F.Cu") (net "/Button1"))
 (via (at 161.215209 30.203422) (size 0.6) (drill 0.3) (layers "F.Cu" "B.Cu") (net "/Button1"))
 (segment (start 193.602 26.409786) (end 193.341214 26.149) (width 0.2) (layer "F.Cu") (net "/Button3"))
 (segment (start 190.614473 29.803422) (end 188.763422 29.803422) (width 0.2) (layer "F.Cu") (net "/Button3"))
 (segment (start 193.341214 26.149) (end 191.738786 26.149) (width 0.2) (layer "F.Cu") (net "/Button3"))
 (segment (start 191.478 28.939895) (end 190.614473 29.803422) (width 0.2) (layer "F.Cu") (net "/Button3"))
 (segment (start 159.85 56.65) (end 184.135 32.365) (width 0.2) (layer "F.Cu") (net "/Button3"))
 (segment (start 191.478 26.409786) (end 191.478 28.939895) (width 0.2) (layer "F.Cu") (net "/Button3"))
 (segment (start 184.135 32.365) (end 190.176895 32.365) (width 0.2) (layer "F.Cu") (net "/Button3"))
 (segment (start 193.602 28.939895) (end 193.602 26.409786) (width 0.2) (layer "F.Cu") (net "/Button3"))
 (segment (start 188.763422 29.803422) (end 187.46 28.5) (width 0.2) (layer "F.Cu") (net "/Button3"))
 (segment (start 159.85 63.96) (end 159.85 56.65) (width 0.2) (layer "F.Cu") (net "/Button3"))
 (segment (start 190.176895 32.365) (end 193.602 28.939895) (width 0.2) (layer "F.Cu") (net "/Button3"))
 (segment (start 191.738786 26.149) (end 191.478 26.409786) (width 0.2) (layer "F.Cu") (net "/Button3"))
 (segment (start 179.84 28.5) (end 180.205457 28.5) (width 0.2) (layer "F.Cu") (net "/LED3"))
 (segment (start 180.205457 28.5) (end 180.667457 28.962) (width 0.2) (layer "F.Cu") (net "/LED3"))
 (via (at 180.667457 28.962) (size 0.6) (drill 0.3) (layers "F.Cu" "B.Cu") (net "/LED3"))
 (segment (start 180.667457 28.962) (end 185.982 34.276543) (width 0.2) (layer "B.Cu") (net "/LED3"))
 (segment (start 185.982 55.632) (end 189.5 59.15) (width 0.2) (layer "B.Cu") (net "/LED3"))
 (segment (start 185.982 34.276543) (end 185.982 55.632) (width 0.2) (layer "B.Cu") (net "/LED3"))
 (segment (start 176.5 67) (end 184.35 59.15) (width 0.2) (layer "F.Cu") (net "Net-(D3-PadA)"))
 (segment (start 184.35 59.15) (end 184.42 59.15) (width 0.2) (layer "F.Cu") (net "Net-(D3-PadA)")))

